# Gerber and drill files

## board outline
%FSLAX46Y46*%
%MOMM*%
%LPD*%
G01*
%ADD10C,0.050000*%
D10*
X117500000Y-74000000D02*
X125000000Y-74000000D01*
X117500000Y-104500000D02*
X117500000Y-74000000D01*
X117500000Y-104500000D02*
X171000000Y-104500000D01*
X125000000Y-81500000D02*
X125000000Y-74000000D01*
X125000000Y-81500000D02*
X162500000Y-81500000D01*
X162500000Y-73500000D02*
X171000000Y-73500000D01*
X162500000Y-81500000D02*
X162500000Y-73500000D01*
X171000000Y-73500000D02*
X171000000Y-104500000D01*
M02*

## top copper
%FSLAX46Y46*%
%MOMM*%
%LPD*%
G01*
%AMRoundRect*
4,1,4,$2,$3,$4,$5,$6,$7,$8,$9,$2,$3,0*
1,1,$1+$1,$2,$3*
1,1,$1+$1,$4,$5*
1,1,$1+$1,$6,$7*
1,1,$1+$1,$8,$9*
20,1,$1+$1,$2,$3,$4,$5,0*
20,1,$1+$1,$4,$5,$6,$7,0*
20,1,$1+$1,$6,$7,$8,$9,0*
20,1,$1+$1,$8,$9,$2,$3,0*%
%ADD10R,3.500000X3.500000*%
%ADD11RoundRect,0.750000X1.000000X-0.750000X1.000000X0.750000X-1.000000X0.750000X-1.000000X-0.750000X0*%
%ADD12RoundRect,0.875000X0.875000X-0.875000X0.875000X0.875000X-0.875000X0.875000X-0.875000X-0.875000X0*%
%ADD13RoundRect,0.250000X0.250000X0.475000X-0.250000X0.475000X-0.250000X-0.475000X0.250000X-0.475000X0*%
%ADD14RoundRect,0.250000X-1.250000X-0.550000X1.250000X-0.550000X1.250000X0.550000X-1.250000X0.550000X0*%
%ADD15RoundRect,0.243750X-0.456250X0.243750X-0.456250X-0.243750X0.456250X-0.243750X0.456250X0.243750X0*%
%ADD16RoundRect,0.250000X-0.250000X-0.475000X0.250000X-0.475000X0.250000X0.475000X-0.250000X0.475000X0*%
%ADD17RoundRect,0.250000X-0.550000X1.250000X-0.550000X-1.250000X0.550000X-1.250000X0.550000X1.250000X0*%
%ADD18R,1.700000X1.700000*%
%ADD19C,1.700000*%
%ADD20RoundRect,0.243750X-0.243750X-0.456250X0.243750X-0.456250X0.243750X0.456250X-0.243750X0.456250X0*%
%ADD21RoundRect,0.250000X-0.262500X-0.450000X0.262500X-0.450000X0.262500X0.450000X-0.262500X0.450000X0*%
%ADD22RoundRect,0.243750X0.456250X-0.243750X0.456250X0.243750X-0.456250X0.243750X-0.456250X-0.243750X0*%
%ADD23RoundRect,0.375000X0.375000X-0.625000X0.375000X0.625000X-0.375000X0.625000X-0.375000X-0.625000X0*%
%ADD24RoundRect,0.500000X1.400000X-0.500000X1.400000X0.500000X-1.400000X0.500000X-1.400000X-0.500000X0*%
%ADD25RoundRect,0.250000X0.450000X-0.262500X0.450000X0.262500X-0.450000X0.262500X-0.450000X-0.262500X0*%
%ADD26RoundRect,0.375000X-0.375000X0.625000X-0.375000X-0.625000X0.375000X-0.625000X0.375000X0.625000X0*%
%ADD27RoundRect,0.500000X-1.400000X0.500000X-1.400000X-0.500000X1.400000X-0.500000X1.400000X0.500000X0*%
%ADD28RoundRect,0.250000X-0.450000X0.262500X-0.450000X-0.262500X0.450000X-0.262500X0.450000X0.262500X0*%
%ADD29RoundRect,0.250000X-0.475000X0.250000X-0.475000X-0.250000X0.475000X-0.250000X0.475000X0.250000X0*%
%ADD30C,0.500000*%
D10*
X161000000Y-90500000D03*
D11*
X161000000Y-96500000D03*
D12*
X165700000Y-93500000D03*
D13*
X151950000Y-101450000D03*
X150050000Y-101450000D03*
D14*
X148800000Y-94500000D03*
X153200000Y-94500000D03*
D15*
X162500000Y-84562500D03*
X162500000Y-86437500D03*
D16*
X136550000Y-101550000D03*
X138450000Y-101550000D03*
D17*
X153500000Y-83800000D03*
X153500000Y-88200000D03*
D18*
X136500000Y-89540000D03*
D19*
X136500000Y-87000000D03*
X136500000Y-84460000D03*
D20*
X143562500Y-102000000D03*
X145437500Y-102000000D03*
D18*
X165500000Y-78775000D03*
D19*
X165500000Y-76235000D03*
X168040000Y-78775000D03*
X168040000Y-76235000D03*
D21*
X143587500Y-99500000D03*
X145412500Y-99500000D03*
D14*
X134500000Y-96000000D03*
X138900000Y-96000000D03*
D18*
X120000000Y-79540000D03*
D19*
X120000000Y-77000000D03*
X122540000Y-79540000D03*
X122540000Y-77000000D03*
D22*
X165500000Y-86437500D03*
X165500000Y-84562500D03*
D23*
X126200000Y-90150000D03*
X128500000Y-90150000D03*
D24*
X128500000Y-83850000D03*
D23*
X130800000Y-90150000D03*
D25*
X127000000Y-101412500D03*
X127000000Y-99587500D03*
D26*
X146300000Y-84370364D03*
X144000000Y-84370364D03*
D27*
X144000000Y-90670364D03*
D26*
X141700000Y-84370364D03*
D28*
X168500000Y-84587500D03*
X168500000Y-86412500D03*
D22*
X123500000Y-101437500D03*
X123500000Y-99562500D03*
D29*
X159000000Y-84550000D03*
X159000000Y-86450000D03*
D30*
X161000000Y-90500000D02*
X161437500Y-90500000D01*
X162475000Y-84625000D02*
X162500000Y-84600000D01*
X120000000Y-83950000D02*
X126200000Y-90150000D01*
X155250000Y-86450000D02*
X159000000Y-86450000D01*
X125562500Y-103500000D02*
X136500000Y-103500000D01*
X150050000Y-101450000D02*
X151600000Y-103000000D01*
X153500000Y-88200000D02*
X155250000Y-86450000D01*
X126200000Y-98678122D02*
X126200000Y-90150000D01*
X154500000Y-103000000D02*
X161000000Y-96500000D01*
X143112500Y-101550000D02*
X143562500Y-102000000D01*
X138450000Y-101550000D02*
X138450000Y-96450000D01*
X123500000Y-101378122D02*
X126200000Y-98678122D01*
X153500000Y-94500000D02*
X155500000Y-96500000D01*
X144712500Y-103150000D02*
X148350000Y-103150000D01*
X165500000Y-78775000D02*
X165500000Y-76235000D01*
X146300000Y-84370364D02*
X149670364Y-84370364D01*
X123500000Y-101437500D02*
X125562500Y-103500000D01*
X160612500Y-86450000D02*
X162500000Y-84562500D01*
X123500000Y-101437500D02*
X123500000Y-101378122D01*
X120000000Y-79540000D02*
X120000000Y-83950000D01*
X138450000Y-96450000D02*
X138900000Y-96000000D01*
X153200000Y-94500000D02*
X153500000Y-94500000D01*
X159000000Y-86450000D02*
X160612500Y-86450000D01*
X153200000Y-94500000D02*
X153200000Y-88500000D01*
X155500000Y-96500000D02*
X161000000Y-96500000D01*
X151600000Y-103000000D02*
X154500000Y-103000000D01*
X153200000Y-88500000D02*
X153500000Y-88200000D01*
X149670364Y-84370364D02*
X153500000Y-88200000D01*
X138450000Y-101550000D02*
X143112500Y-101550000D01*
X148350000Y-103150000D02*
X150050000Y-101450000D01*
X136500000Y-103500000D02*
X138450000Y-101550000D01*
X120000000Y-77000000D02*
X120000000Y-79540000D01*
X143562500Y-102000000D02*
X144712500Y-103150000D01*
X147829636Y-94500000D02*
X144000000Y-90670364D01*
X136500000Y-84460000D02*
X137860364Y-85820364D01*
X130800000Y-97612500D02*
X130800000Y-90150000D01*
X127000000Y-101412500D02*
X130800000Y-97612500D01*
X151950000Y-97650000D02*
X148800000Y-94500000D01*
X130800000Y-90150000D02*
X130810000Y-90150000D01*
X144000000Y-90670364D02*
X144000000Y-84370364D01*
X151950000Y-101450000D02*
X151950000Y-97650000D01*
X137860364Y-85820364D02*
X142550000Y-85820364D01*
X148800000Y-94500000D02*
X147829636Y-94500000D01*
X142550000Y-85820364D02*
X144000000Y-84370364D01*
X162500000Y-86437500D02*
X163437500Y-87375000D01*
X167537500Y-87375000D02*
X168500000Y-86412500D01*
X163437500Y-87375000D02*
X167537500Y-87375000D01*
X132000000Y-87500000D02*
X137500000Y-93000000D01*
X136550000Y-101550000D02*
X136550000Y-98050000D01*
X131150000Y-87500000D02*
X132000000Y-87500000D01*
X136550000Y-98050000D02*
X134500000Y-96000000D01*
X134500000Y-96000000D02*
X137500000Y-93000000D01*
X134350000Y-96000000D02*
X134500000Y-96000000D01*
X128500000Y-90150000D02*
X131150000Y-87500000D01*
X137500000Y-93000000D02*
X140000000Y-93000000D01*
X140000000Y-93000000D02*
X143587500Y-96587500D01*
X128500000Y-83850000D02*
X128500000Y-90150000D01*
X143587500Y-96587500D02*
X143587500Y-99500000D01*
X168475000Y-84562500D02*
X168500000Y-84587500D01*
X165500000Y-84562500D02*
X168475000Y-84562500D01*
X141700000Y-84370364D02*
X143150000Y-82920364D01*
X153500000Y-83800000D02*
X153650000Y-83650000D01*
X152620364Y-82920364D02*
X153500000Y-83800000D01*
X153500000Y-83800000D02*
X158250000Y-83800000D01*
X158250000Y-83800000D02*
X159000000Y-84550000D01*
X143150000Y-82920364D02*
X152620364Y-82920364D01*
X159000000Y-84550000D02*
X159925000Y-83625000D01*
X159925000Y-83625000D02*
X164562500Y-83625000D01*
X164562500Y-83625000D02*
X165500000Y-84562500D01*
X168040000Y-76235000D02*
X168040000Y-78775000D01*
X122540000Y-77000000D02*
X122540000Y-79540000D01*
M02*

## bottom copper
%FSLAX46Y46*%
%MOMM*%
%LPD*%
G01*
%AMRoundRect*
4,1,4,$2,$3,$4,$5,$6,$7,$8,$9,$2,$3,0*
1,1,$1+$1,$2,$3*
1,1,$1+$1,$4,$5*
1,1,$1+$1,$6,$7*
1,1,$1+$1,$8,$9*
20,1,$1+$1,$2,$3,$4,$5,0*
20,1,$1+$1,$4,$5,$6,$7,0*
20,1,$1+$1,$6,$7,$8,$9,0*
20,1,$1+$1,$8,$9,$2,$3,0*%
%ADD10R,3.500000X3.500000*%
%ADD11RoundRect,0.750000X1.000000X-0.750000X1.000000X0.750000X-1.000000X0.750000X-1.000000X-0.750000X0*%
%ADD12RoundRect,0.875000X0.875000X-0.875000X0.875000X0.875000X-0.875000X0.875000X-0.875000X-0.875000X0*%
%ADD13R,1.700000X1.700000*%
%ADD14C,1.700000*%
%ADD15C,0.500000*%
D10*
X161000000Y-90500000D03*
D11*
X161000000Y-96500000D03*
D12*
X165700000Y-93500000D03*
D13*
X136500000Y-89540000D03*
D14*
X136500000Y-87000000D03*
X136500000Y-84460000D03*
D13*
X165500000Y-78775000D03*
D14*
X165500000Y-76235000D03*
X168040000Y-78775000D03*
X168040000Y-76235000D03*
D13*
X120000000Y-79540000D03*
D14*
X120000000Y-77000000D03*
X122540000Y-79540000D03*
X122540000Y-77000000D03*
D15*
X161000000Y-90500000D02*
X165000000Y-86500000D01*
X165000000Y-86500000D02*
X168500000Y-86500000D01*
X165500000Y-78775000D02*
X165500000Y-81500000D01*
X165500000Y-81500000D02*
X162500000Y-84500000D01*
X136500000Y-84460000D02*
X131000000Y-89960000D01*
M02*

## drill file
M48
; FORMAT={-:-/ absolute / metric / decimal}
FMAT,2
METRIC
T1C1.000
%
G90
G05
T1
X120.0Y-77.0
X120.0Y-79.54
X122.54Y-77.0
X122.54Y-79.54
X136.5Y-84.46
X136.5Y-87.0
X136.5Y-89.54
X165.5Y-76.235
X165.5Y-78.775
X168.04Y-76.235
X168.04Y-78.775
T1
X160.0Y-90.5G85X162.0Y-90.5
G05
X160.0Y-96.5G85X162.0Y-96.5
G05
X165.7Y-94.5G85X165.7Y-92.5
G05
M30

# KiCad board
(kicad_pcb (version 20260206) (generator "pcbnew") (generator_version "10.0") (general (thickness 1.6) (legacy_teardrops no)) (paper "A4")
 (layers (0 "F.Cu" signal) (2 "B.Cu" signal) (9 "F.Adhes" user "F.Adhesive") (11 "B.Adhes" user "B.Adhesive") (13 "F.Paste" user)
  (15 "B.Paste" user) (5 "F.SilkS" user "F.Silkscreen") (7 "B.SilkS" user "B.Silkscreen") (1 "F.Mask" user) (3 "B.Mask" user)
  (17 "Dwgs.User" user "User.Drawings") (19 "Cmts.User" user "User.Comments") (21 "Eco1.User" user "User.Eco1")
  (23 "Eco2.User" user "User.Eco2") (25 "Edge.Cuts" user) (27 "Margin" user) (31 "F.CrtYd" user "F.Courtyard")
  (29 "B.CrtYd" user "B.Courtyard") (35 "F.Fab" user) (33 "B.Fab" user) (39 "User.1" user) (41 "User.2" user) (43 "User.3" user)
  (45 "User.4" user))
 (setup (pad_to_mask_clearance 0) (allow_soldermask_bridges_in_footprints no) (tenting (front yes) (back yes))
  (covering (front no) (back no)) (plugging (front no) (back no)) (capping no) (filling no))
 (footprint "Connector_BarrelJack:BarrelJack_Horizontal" (layer "F.Cu") (at 161 90.5 90)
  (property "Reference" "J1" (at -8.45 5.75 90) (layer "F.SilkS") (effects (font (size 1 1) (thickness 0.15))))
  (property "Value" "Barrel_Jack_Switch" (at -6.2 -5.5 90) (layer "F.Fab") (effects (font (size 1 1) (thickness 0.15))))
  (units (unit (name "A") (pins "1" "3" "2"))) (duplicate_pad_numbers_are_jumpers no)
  (pad "1" thru_hole rect (at 0 0 90) (size 3.5 3.5) (drill oval 1 3) (layers "*.Cu" "*.Mask") (remove_unused_layers no)
   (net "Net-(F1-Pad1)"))
  (pad "2" thru_hole roundrect (at -6 0 90) (size 3 3.5) (drill oval 1 3) (layers "*.Cu" "*.Mask") (remove_unused_layers no)
   (roundrect_rratio 0.25) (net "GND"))
  (pad "3" thru_hole roundrect (at -3 4.7 90) (size 3.5 3.5) (drill oval 3 1) (layers "*.Cu" "*.Mask") (remove_unused_layers no)
   (roundrect_rratio 0.25) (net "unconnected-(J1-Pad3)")))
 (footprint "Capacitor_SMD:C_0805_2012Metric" (layer "F.Cu") (at 151 101.45 180)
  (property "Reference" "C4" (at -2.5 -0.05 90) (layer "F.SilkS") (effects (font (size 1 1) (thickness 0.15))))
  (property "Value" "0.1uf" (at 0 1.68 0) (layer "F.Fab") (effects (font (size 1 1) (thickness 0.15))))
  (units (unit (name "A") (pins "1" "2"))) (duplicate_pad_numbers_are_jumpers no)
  (pad "1" smd roundrect (at -0.95 0 180) (size 1 1.45) (layers "F.Cu" "F.Mask" "F.Paste") (roundrect_rratio 0.25) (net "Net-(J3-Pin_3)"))
  (pad "2" smd roundrect (at 0.95 0 180) (size 1 1.45) (layers "F.Cu" "F.Mask" "F.Paste") (roundrect_rratio 0.25) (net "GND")))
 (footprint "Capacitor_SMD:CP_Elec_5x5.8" (layer "F.Cu") (at 151 94.5)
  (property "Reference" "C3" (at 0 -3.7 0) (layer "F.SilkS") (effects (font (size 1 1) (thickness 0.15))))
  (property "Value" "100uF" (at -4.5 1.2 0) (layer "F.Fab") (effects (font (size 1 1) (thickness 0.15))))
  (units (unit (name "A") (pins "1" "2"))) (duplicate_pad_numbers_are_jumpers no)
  (pad "1" smd roundrect (at -2.2 0) (size 3 1.6) (layers "F.Cu" "F.Mask" "F.Paste") (roundrect_rratio 0.15625) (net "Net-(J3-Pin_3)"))
  (pad "2" smd roundrect (at 2.2 0) (size 3 1.6) (layers "F.Cu" "F.Mask" "F.Paste") (roundrect_rratio 0.15625) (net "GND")))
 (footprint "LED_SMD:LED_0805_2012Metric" (layer "F.Cu") (at 162.5 85.5 -90)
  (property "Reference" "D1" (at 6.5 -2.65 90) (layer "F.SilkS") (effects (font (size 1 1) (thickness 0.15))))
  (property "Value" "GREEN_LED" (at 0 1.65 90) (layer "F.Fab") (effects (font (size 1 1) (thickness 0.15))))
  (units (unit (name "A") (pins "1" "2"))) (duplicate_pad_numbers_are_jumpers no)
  (pad "1" smd roundrect (at -0.9375 0 270) (size 0.975 1.4) (layers "F.Cu" "F.Mask" "F.Paste") (roundrect_rratio 0.25) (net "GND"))
  (pad "2" smd roundrect (at 0.9375 0 270) (size 0.975 1.4) (layers "F.Cu" "F.Mask" "F.Paste") (roundrect_rratio 0.25) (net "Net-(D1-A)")))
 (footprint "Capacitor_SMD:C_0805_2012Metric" (layer "F.Cu") (at 137.5 101.55)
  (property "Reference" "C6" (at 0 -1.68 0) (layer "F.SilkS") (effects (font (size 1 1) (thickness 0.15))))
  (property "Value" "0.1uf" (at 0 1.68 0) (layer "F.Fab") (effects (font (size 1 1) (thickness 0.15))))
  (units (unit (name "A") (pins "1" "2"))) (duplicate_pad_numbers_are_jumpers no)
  (pad "1" smd roundrect (at -0.95 0) (size 1 1.45) (layers "F.Cu" "F.Mask" "F.Paste") (roundrect_rratio 0.25) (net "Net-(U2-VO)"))
  (pad "2" smd roundrect (at 0.95 0) (size 1 1.45) (layers "F.Cu" "F.Mask" "F.Paste") (roundrect_rratio 0.25) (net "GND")))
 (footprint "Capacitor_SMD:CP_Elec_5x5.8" (layer "F.Cu") (at 153.5 86 -90)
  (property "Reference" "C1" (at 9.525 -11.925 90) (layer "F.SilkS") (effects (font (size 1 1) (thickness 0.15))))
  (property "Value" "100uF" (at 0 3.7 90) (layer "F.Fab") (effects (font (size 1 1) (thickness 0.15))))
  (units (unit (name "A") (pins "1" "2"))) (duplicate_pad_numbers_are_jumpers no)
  (pad "1" smd roundrect (at -2.2 0 270) (size 3 1.6) (layers "F.Cu" "F.Mask" "F.Paste") (roundrect_rratio 0.15625) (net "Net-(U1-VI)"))
  (pad "2" smd roundrect (at 2.2 0 270) (size 3 1.6) (layers "F.Cu" "F.Mask" "F.Paste") (roundrect_rratio 0.15625) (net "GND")))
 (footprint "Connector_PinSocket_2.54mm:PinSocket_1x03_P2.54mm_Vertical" (layer "F.Cu") (at 136.5 89.54 180)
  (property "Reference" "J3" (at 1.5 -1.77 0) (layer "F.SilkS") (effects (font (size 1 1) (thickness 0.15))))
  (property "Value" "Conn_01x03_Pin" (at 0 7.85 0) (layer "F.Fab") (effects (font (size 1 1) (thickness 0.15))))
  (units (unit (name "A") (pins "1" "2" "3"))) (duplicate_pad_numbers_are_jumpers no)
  (pad "1" thru_hole rect (at 0 0 180) (size 1.7 1.7) (drill 1) (layers "*.Cu" "*.Mask") (remove_unused_layers no)
   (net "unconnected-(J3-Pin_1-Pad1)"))
  (pad "2" thru_hole circle (at 0 2.54 180) (size 1.7 1.7) (drill 1) (layers "*.Cu" "*.Mask") (remove_unused_layers no)
   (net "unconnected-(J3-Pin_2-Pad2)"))
  (pad "3" thru_hole circle (at 0 5.08 180) (size 1.7 1.7) (drill 1) (layers "*.Cu" "*.Mask") (remove_unused_layers no)
   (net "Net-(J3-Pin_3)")))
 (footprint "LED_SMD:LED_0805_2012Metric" (layer "F.Cu") (at 144.5 102)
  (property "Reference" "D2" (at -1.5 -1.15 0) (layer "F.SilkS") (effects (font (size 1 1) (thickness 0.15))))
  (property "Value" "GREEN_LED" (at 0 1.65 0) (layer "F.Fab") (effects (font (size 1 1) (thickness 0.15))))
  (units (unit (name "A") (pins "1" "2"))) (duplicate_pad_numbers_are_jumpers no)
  (pad "1" smd roundrect (at -0.9375 0) (size 0.975 1.4) (layers "F.Cu" "F.Mask" "F.Paste") (roundrect_rratio 0.25) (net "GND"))
  (pad "2" smd roundrect (at 0.9375 0) (size 0.975 1.4) (layers "F.Cu" "F.Mask" "F.Paste") (roundrect_rratio 0.25) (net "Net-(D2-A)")))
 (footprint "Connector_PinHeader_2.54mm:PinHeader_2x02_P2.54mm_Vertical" (layer "F.Cu") (at 165.5 78.775 90)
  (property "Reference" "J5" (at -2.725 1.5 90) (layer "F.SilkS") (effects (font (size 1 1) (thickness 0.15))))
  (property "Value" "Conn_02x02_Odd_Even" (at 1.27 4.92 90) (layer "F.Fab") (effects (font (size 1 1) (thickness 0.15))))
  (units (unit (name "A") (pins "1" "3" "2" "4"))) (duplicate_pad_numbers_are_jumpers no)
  (pad "1" thru_hole rect (at 0 0 90) (size 1.7 1.7) (drill 1) (layers "*.Cu" "*.Mask") (remove_unused_layers no) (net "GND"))
  (pad "2" thru_hole circle (at 2.54 0 90) (size 1.7 1.7) (drill 1) (layers "*.Cu" "*.Mask") (remove_unused_layers no) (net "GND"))
  (pad "3" thru_hole circle (at 0 2.54 90) (size 1.7 1.7) (drill 1) (layers "*.Cu" "*.Mask") (remove_unused_layers no)
   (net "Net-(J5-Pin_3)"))
  (pad "4" thru_hole circle (at 2.54 2.54 90) (size 1.7 1.7) (drill 1) (layers "*.Cu" "*.Mask") (remove_unused_layers no)
   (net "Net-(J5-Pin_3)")))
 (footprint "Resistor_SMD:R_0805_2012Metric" (layer "F.Cu") (at 144.5 99.5)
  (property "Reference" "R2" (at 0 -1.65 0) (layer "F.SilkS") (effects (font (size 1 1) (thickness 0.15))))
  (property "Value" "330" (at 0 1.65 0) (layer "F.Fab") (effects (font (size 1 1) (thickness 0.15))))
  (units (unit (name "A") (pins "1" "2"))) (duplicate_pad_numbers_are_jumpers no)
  (pad "1" smd roundrect (at -0.9125 0) (size 1.025 1.4) (layers "F.Cu" "F.Mask" "F.Paste") (roundrect_rratio 0.243902) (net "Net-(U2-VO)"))
  (pad "2" smd roundrect (at 0.9125 0) (size 1.025 1.4) (layers "F.Cu" "F.Mask" "F.Paste") (roundrect_rratio 0.243902) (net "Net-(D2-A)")))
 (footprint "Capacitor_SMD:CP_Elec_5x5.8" (layer "F.Cu") (at 136.7 96)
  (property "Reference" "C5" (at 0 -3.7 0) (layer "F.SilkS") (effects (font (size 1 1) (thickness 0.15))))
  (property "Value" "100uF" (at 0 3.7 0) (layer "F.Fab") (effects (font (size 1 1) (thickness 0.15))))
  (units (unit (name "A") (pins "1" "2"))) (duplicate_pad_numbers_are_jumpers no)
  (pad "1" smd roundrect (at -2.2 0) (size 3 1.6) (layers "F.Cu" "F.Mask" "F.Paste") (roundrect_rratio 0.15625) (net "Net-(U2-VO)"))
  (pad "2" smd roundrect (at 2.2 0) (size 3 1.6) (layers "F.Cu" "F.Mask" "F.Paste") (roundrect_rratio 0.15625) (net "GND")))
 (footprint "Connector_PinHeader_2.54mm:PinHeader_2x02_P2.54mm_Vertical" (layer "F.Cu") (at 120 79.54 90)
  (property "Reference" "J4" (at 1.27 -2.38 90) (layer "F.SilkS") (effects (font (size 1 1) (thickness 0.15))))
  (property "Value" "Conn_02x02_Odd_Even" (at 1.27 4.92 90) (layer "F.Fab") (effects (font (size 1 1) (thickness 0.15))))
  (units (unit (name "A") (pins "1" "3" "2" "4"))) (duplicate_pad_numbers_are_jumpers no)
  (pad "1" thru_hole rect (at 0 0 90) (size 1.7 1.7) (drill 1) (layers "*.Cu" "*.Mask") (remove_unused_layers no) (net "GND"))
  (pad "2" thru_hole circle (at 2.54 0 90) (size 1.7 1.7) (drill 1) (layers "*.Cu" "*.Mask") (remove_unused_layers no) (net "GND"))
  (pad "3" thru_hole circle (at 0 2.54 90) (size 1.7 1.7) (drill 1) (layers "*.Cu" "*.Mask") (remove_unused_layers no)
   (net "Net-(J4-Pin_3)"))
  (pad "4" thru_hole circle (at 2.54 2.54 90) (size 1.7 1.7) (drill 1) (layers "*.Cu" "*.Mask") (remove_unused_layers no)
   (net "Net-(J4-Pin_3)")))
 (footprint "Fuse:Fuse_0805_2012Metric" (layer "F.Cu") (at 165.5 85.5 90)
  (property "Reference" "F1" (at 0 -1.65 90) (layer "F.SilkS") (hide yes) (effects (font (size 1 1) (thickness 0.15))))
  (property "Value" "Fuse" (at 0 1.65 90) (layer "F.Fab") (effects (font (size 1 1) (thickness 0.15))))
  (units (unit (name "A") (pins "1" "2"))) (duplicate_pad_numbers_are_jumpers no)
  (pad "1" smd roundrect (at -0.9375 0 90) (size 0.975 1.4) (layers "F.Cu" "F.Mask" "F.Paste") (roundrect_rratio 0.25) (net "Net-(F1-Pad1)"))
  (pad "2" smd roundrect (at 0.9375 0 90) (size 0.975 1.4) (layers "F.Cu" "F.Mask" "F.Paste") (roundrect_rratio 0.25) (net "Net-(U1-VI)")))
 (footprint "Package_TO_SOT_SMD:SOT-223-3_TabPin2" (layer "F.Cu") (at 128.5 87 90)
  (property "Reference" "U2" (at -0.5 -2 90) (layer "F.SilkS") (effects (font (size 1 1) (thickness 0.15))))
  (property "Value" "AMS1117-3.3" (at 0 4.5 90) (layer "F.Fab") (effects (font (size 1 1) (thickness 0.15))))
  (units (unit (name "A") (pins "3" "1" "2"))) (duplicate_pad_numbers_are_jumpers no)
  (pad "1" smd roundrect (at -3.15 -2.3 90) (size 2 1.5) (layers "F.Cu" "F.Mask" "F.Paste") (roundrect_rratio 0.25) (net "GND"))
  (pad "2" smd roundrect (at -3.15 0 90) (size 2 1.5) (layers "F.Cu" "F.Mask" "F.Paste") (roundrect_rratio 0.25) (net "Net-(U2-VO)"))
  (pad "2" smd roundrect (at 3.15 0 90) (size 2 3.8) (layers "F.Cu" "F.Mask" "F.Paste") (roundrect_rratio 0.25) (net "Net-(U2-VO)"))
  (pad "3" smd roundrect (at -3.15 2.3 90) (size 2 1.5) (layers "F.Cu" "F.Mask" "F.Paste") (roundrect_rratio 0.25) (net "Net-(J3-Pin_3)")))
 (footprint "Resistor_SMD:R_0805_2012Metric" (layer "F.Cu") (at 127 100.5 90)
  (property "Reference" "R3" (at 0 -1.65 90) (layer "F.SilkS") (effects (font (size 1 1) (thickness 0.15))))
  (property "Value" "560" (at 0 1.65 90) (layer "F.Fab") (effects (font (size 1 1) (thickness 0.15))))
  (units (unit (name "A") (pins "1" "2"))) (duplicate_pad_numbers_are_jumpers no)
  (pad "1" smd roundrect (at -0.9125 0 90) (size 1.025 1.4) (layers "F.Cu" "F.Mask" "F.Paste") (roundrect_rratio 0.243902)
   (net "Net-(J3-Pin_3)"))
  (pad "2" smd roundrect (at 0.9125 0 90) (size 1.025 1.4) (layers "F.Cu" "F.Mask" "F.Paste") (roundrect_rratio 0.243902) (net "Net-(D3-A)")))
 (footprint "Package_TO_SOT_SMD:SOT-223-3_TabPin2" (layer "F.Cu") (at 144 87.520364 -90)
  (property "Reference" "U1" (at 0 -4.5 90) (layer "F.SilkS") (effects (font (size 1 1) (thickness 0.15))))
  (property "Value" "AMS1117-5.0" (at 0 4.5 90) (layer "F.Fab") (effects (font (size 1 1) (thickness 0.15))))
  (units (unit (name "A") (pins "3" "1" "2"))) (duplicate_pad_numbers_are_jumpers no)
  (pad "1" smd roundrect (at -3.15 -2.3 270) (size 2 1.5) (layers "F.Cu" "F.Mask" "F.Paste") (roundrect_rratio 0.25) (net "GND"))
  (pad "2" smd roundrect (at -3.15 0 270) (size 2 1.5) (layers "F.Cu" "F.Mask" "F.Paste") (roundrect_rratio 0.25) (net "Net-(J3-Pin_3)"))
  (pad "2" smd roundrect (at 3.15 0 270) (size 2 3.8) (layers "F.Cu" "F.Mask" "F.Paste") (roundrect_rratio 0.25) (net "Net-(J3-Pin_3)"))
  (pad "3" smd roundrect (at -3.15 2.3 270) (size 2 1.5) (layers "F.Cu" "F.Mask" "F.Paste") (roundrect_rratio 0.25) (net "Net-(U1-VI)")))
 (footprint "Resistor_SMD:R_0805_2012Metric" (layer "F.Cu") (at 168.5 85.5 -90)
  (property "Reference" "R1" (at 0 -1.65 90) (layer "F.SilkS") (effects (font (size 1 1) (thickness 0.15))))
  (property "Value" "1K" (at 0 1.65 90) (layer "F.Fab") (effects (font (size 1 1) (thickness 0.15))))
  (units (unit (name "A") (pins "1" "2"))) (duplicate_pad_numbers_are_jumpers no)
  (pad "1" smd roundrect (at -0.9125 0 270) (size 1.025 1.4) (layers "F.Cu" "F.Mask" "F.Paste") (roundrect_rratio 0.243902)
   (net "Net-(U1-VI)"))
  (pad "2" smd roundrect (at 0.9125 0 270) (size 1.025 1.4) (layers "F.Cu" "F.Mask" "F.Paste") (roundrect_rratio 0.243902)
   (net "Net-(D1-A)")))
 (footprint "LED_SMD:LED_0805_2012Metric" (layer "F.Cu") (at 123.5 100.5 90)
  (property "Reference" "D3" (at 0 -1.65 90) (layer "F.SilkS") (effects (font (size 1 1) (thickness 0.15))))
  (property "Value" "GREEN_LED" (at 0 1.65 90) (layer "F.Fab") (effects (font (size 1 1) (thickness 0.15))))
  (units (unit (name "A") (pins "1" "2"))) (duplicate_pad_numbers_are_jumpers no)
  (pad "1" smd roundrect (at -0.9375 0 90) (size 0.975 1.4) (layers "F.Cu" "F.Mask" "F.Paste") (roundrect_rratio 0.25) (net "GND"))
  (pad "2" smd roundrect (at 0.9375 0 90) (size 0.975 1.4) (layers "F.Cu" "F.Mask" "F.Paste") (roundrect_rratio 0.25) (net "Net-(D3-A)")))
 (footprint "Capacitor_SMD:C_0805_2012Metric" (layer "F.Cu") (at 159 85.5 -90)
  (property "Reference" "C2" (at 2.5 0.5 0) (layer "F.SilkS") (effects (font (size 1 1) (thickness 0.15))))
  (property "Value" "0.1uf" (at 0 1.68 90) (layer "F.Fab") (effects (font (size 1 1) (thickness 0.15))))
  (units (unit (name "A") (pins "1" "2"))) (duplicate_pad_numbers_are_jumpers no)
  (pad "1" smd roundrect (at -0.95 0 270) (size 1 1.45) (layers "F.Cu" "F.Mask" "F.Paste") (roundrect_rratio 0.25) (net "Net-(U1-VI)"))
  (pad "2" smd roundrect (at 0.95 0 270) (size 1 1.45) (layers "F.Cu" "F.Mask" "F.Paste") (roundrect_rratio 0.25) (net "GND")))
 (gr_line (start 117.5 74) (end 125 74) (stroke (width 0.05) (type default)) (layer "Edge.Cuts"))
 (gr_line (start 117.5 104.5) (end 117.5 74) (stroke (width 0.05) (type default)) (layer "Edge.Cuts"))
 (gr_line (start 117.5 104.5) (end 171 104.5) (stroke (width 0.05) (type default)) (layer "Edge.Cuts"))
 (gr_line (start 125 81.5) (end 125 74) (stroke (width 0.05) (type default)) (layer "Edge.Cuts"))
 (gr_line (start 125 81.5) (end 162.5 81.5) (stroke (width 0.05) (type default)) (layer "Edge.Cuts"))
 (gr_line (start 162.5 73.5) (end 171 73.5) (stroke (width 0.05) (type default)) (layer "Edge.Cuts"))
 (gr_line (start 162.5 81.5) (end 162.5 73.5) (stroke (width 0.05) (type default)) (layer "Edge.Cuts"))
 (gr_line (start 171 73.5) (end 171 104.5) (stroke (width 0.05) (type default)) (layer "Edge.Cuts"))
 (segment (start 161 90.5) (end 161.4375 90.5) (width 0.5) (layer "F.Cu") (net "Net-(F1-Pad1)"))
 (segment (start 161 90.5) (end 165 86.5) (width 0.5) (layer "B.Cu") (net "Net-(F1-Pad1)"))
 (segment (start 165 86.5) (end 168.5 86.5) (width 0.5) (layer "B.Cu") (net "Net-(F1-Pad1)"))
 (segment (start 162.475 84.625) (end 162.5 84.6) (width 0.5) (layer "F.Cu") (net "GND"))
 (segment (start 120 83.95) (end 126.2 90.15) (width 0.5) (layer "F.Cu") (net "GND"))
 (segment (start 155.25 86.45) (end 159 86.45) (width 0.5) (layer "F.Cu") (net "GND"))
 (segment (start 125.5625 103.5) (end 136.5 103.5) (width 0.5) (layer "F.Cu") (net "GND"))
 (segment (start 150.05 101.45) (end 151.6 103) (width 0.5) (layer "F.Cu") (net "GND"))
 (segment (start 153.5 88.2) (end 155.25 86.45) (width 0.5) (layer "F.Cu") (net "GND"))
 (segment (start 126.2 98.678122) (end 126.2 90.15) (width 0.5) (layer "F.Cu") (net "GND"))
 (segment (start 154.5 103) (end 161 96.5) (width 0.5) (layer "F.Cu") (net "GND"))
 (segment (start 143.1125 101.55) (end 143.5625 102) (width 0.5) (layer "F.Cu") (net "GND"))
 (segment (start 138.45 101.55) (end 138.45 96.45) (width 0.5) (layer "F.Cu") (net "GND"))
 (segment (start 123.5 101.378122) (end 126.2 98.678122) (width 0.5) (layer "F.Cu") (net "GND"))
 (segment (start 153.5 94.5) (end 155.5 96.5) (width 0.5) (layer "F.Cu") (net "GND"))
 (segment (start 144.7125 103.15) (end 148.35 103.15) (width 0.5) (layer "F.Cu") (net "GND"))
 (segment (start 165.5 78.775) (end 165.5 76.235) (width 0.5) (layer "F.Cu") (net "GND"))
 (segment (start 146.3 84.370364) (end 149.670364 84.370364) (width 0.5) (layer "F.Cu") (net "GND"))
 (segment (start 123.5 101.4375) (end 125.5625 103.5) (width 0.5) (layer "F.Cu") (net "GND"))
 (segment (start 160.6125 86.45) (end 162.5 84.5625) (width 0.5) (layer "F.Cu") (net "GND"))
 (segment (start 123.5 101.4375) (end 123.5 101.378122) (width 0.5) (layer "F.Cu") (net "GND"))
 (segment (start 120 79.54) (end 120 83.95) (width 0.5) (layer "F.Cu") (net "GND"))
 (segment (start 138.45 96.45) (end 138.9 96) (width 0.5) (layer "F.Cu") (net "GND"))
 (segment (start 153.2 94.5) (end 153.5 94.5) (width 0.5) (layer "F.Cu") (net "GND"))
 (segment (start 159 86.45) (end 160.6125 86.45) (width 0.5) (layer "F.Cu") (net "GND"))
 (segment (start 153.2 94.5) (end 153.2 88.5) (width 0.5) (layer "F.Cu") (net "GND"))
 (segment (start 155.5 96.5) (end 161 96.5) (width 0.5) (layer "F.Cu") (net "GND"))
 (segment (start 151.6 103) (end 154.5 103) (width 0.5) (layer "F.Cu") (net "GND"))
 (segment (start 153.2 88.5) (end 153.5 88.2) (width 0.5) (layer "F.Cu") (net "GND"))
 (segment (start 149.670364 84.370364) (end 153.5 88.2) (width 0.5) (layer "F.Cu") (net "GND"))
 (segment (start 138.45 101.55) (end 143.1125 101.55) (width 0.5) (layer "F.Cu") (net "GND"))
 (segment (start 148.35 103.15) (end 150.05 101.45) (width 0.5) (layer "F.Cu") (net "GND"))
 (segment (start 136.5 103.5) (end 138.45 101.55) (width 0.5) (layer "F.Cu") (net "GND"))
 (segment (start 120 77) (end 120 79.54) (width 0.5) (layer "F.Cu") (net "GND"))
 (segment (start 143.5625 102) (end 144.7125 103.15) (width 0.5) (layer "F.Cu") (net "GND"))
 (segment (start 165.5 78.775) (end 165.5 81.5) (width 0.5) (layer "B.Cu") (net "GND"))
 (segment (start 165.5 81.5) (end 162.5 84.5) (width 0.5) (layer "B.Cu") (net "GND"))
 (segment (start 147.829636 94.5) (end 144 90.670364) (width 0.5) (layer "F.Cu") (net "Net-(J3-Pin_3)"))
 (segment (start 136.5 84.46) (end 137.860364 85.820364) (width 0.5) (layer "F.Cu") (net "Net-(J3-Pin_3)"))
 (segment (start 130.8 97.6125) (end 130.8 90.15) (width 0.5) (layer "F.Cu") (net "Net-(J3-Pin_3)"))
 (segment (start 127 101.4125) (end 130.8 97.6125) (width 0.5) (layer "F.Cu") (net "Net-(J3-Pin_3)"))
 (segment (start 151.95 97.65) (end 148.8 94.5) (width 0.5) (layer "F.Cu") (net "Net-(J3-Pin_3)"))
 (segment (start 130.8 90.15) (end 130.81 90.15) (width 0.5) (layer "F.Cu") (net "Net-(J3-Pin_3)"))
 (segment (start 144 90.670364) (end 144 84.370364) (width 0.5) (layer "F.Cu") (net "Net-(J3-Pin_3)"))
 (segment (start 151.95 101.45) (end 151.95 97.65) (width 0.5) (layer "F.Cu") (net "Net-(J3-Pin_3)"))
 (segment (start 137.860364 85.820364) (end 142.55 85.820364) (width 0.5) (layer "F.Cu") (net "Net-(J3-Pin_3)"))
 (segment (start 148.8 94.5) (end 147.829636 94.5) (width 0.5) (layer "F.Cu") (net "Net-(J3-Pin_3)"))
 (segment (start 142.55 85.820364) (end 144 84.370364) (width 0.5) (layer "F.Cu") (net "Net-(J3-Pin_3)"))
 (segment (start 136.5 84.46) (end 131 89.96) (width 0.5) (layer "B.Cu") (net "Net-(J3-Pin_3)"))
 (segment (start 162.5 86.4375) (end 163.4375 87.375) (width 0.5) (layer "F.Cu") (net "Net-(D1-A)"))
 (segment (start 167.5375 87.375) (end 168.5 86.4125) (width 0.5) (layer "F.Cu") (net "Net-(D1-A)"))
 (segment (start 163.4375 87.375) (end 167.5375 87.375) (width 0.5) (layer "F.Cu") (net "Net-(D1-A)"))
 (segment (start 132 87.5) (end 137.5 93) (width 0.5) (layer "F.Cu") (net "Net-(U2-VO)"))
 (segment (start 136.55 101.55) (end 136.55 98.05) (width 0.5) (layer "F.Cu") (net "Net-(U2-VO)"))
 (segment (start 131.15 87.5) (end 132 87.5) (width 0.5) (layer "F.Cu") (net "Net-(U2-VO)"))
 (segment (start 136.55 98.05) (end 134.5 96) (width 0.5) (layer "F.Cu") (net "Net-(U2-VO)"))
 (segment (start 134.5 96) (end 137.5 93) (width 0.5) (layer "F.Cu") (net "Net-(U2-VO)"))
 (segment (start 134.35 96) (end 134.5 96) (width 0.5) (layer "F.Cu") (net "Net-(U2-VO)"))
 (segment (start 128.5 90.15) (end 131.15 87.5) (width 0.5) (layer "F.Cu") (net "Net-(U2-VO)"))
 (segment (start 137.5 93) (end 140 93) (width 0.5) (layer "F.Cu") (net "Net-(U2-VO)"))
 (segment (start 140 93) (end 143.5875 96.5875) (width 0.5) (layer "F.Cu") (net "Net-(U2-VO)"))
 (segment (start 128.5 83.85) (end 128.5 90.15) (width 0.5) (layer "F.Cu") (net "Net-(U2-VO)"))
 (segment (start 143.5875 96.5875) (end 143.5875 99.5) (width 0.5) (layer "F.Cu") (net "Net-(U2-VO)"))
 (segment (start 168.475 84.5625) (end 168.5 84.5875) (width 0.5) (layer "F.Cu") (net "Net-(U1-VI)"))
 (segment (start 165.5 84.5625) (end 168.475 84.5625) (width 0.5) (layer "F.Cu") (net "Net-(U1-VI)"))
 (segment (start 141.7 84.370364) (end 143.15 82.920364) (width 0.5) (layer "F.Cu") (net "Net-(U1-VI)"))
 (segment (start 153.5 83.8) (end 153.65 83.65) (width 0.5) (layer "F.Cu") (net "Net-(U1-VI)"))
 (segment (start 152.620364 82.920364) (end 153.5 83.8) (width 0.5) (layer "F.Cu") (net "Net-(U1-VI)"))
 (segment (start 153.5 83.8) (end 158.25 83.8) (width 0.5) (layer "F.Cu") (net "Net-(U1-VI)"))
 (segment (start 158.25 83.8) (end 159 84.55) (width 0.5) (layer "F.Cu") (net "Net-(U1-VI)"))
 (segment (start 143.15 82.920364) (end 152.620364 82.920364) (width 0.5) (layer "F.Cu") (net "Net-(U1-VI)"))
 (segment (start 159 84.55) (end 159.925 83.625) (width 0.5) (layer "F.Cu") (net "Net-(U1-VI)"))
 (segment (start 159.925 83.625) (end 164.5625 83.625) (width 0.5) (layer "F.Cu") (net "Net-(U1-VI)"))
 (segment (start 164.5625 83.625) (end 165.5 84.5625) (width 0.5) (layer "F.Cu") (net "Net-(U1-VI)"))
 (segment (start 168.04 76.235) (end 168.04 78.775) (width 0.5) (layer "F.Cu") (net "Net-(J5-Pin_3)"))
 (segment (start 122.54 77) (end 122.54 79.54) (width 0.5) (layer "F.Cu") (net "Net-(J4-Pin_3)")))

